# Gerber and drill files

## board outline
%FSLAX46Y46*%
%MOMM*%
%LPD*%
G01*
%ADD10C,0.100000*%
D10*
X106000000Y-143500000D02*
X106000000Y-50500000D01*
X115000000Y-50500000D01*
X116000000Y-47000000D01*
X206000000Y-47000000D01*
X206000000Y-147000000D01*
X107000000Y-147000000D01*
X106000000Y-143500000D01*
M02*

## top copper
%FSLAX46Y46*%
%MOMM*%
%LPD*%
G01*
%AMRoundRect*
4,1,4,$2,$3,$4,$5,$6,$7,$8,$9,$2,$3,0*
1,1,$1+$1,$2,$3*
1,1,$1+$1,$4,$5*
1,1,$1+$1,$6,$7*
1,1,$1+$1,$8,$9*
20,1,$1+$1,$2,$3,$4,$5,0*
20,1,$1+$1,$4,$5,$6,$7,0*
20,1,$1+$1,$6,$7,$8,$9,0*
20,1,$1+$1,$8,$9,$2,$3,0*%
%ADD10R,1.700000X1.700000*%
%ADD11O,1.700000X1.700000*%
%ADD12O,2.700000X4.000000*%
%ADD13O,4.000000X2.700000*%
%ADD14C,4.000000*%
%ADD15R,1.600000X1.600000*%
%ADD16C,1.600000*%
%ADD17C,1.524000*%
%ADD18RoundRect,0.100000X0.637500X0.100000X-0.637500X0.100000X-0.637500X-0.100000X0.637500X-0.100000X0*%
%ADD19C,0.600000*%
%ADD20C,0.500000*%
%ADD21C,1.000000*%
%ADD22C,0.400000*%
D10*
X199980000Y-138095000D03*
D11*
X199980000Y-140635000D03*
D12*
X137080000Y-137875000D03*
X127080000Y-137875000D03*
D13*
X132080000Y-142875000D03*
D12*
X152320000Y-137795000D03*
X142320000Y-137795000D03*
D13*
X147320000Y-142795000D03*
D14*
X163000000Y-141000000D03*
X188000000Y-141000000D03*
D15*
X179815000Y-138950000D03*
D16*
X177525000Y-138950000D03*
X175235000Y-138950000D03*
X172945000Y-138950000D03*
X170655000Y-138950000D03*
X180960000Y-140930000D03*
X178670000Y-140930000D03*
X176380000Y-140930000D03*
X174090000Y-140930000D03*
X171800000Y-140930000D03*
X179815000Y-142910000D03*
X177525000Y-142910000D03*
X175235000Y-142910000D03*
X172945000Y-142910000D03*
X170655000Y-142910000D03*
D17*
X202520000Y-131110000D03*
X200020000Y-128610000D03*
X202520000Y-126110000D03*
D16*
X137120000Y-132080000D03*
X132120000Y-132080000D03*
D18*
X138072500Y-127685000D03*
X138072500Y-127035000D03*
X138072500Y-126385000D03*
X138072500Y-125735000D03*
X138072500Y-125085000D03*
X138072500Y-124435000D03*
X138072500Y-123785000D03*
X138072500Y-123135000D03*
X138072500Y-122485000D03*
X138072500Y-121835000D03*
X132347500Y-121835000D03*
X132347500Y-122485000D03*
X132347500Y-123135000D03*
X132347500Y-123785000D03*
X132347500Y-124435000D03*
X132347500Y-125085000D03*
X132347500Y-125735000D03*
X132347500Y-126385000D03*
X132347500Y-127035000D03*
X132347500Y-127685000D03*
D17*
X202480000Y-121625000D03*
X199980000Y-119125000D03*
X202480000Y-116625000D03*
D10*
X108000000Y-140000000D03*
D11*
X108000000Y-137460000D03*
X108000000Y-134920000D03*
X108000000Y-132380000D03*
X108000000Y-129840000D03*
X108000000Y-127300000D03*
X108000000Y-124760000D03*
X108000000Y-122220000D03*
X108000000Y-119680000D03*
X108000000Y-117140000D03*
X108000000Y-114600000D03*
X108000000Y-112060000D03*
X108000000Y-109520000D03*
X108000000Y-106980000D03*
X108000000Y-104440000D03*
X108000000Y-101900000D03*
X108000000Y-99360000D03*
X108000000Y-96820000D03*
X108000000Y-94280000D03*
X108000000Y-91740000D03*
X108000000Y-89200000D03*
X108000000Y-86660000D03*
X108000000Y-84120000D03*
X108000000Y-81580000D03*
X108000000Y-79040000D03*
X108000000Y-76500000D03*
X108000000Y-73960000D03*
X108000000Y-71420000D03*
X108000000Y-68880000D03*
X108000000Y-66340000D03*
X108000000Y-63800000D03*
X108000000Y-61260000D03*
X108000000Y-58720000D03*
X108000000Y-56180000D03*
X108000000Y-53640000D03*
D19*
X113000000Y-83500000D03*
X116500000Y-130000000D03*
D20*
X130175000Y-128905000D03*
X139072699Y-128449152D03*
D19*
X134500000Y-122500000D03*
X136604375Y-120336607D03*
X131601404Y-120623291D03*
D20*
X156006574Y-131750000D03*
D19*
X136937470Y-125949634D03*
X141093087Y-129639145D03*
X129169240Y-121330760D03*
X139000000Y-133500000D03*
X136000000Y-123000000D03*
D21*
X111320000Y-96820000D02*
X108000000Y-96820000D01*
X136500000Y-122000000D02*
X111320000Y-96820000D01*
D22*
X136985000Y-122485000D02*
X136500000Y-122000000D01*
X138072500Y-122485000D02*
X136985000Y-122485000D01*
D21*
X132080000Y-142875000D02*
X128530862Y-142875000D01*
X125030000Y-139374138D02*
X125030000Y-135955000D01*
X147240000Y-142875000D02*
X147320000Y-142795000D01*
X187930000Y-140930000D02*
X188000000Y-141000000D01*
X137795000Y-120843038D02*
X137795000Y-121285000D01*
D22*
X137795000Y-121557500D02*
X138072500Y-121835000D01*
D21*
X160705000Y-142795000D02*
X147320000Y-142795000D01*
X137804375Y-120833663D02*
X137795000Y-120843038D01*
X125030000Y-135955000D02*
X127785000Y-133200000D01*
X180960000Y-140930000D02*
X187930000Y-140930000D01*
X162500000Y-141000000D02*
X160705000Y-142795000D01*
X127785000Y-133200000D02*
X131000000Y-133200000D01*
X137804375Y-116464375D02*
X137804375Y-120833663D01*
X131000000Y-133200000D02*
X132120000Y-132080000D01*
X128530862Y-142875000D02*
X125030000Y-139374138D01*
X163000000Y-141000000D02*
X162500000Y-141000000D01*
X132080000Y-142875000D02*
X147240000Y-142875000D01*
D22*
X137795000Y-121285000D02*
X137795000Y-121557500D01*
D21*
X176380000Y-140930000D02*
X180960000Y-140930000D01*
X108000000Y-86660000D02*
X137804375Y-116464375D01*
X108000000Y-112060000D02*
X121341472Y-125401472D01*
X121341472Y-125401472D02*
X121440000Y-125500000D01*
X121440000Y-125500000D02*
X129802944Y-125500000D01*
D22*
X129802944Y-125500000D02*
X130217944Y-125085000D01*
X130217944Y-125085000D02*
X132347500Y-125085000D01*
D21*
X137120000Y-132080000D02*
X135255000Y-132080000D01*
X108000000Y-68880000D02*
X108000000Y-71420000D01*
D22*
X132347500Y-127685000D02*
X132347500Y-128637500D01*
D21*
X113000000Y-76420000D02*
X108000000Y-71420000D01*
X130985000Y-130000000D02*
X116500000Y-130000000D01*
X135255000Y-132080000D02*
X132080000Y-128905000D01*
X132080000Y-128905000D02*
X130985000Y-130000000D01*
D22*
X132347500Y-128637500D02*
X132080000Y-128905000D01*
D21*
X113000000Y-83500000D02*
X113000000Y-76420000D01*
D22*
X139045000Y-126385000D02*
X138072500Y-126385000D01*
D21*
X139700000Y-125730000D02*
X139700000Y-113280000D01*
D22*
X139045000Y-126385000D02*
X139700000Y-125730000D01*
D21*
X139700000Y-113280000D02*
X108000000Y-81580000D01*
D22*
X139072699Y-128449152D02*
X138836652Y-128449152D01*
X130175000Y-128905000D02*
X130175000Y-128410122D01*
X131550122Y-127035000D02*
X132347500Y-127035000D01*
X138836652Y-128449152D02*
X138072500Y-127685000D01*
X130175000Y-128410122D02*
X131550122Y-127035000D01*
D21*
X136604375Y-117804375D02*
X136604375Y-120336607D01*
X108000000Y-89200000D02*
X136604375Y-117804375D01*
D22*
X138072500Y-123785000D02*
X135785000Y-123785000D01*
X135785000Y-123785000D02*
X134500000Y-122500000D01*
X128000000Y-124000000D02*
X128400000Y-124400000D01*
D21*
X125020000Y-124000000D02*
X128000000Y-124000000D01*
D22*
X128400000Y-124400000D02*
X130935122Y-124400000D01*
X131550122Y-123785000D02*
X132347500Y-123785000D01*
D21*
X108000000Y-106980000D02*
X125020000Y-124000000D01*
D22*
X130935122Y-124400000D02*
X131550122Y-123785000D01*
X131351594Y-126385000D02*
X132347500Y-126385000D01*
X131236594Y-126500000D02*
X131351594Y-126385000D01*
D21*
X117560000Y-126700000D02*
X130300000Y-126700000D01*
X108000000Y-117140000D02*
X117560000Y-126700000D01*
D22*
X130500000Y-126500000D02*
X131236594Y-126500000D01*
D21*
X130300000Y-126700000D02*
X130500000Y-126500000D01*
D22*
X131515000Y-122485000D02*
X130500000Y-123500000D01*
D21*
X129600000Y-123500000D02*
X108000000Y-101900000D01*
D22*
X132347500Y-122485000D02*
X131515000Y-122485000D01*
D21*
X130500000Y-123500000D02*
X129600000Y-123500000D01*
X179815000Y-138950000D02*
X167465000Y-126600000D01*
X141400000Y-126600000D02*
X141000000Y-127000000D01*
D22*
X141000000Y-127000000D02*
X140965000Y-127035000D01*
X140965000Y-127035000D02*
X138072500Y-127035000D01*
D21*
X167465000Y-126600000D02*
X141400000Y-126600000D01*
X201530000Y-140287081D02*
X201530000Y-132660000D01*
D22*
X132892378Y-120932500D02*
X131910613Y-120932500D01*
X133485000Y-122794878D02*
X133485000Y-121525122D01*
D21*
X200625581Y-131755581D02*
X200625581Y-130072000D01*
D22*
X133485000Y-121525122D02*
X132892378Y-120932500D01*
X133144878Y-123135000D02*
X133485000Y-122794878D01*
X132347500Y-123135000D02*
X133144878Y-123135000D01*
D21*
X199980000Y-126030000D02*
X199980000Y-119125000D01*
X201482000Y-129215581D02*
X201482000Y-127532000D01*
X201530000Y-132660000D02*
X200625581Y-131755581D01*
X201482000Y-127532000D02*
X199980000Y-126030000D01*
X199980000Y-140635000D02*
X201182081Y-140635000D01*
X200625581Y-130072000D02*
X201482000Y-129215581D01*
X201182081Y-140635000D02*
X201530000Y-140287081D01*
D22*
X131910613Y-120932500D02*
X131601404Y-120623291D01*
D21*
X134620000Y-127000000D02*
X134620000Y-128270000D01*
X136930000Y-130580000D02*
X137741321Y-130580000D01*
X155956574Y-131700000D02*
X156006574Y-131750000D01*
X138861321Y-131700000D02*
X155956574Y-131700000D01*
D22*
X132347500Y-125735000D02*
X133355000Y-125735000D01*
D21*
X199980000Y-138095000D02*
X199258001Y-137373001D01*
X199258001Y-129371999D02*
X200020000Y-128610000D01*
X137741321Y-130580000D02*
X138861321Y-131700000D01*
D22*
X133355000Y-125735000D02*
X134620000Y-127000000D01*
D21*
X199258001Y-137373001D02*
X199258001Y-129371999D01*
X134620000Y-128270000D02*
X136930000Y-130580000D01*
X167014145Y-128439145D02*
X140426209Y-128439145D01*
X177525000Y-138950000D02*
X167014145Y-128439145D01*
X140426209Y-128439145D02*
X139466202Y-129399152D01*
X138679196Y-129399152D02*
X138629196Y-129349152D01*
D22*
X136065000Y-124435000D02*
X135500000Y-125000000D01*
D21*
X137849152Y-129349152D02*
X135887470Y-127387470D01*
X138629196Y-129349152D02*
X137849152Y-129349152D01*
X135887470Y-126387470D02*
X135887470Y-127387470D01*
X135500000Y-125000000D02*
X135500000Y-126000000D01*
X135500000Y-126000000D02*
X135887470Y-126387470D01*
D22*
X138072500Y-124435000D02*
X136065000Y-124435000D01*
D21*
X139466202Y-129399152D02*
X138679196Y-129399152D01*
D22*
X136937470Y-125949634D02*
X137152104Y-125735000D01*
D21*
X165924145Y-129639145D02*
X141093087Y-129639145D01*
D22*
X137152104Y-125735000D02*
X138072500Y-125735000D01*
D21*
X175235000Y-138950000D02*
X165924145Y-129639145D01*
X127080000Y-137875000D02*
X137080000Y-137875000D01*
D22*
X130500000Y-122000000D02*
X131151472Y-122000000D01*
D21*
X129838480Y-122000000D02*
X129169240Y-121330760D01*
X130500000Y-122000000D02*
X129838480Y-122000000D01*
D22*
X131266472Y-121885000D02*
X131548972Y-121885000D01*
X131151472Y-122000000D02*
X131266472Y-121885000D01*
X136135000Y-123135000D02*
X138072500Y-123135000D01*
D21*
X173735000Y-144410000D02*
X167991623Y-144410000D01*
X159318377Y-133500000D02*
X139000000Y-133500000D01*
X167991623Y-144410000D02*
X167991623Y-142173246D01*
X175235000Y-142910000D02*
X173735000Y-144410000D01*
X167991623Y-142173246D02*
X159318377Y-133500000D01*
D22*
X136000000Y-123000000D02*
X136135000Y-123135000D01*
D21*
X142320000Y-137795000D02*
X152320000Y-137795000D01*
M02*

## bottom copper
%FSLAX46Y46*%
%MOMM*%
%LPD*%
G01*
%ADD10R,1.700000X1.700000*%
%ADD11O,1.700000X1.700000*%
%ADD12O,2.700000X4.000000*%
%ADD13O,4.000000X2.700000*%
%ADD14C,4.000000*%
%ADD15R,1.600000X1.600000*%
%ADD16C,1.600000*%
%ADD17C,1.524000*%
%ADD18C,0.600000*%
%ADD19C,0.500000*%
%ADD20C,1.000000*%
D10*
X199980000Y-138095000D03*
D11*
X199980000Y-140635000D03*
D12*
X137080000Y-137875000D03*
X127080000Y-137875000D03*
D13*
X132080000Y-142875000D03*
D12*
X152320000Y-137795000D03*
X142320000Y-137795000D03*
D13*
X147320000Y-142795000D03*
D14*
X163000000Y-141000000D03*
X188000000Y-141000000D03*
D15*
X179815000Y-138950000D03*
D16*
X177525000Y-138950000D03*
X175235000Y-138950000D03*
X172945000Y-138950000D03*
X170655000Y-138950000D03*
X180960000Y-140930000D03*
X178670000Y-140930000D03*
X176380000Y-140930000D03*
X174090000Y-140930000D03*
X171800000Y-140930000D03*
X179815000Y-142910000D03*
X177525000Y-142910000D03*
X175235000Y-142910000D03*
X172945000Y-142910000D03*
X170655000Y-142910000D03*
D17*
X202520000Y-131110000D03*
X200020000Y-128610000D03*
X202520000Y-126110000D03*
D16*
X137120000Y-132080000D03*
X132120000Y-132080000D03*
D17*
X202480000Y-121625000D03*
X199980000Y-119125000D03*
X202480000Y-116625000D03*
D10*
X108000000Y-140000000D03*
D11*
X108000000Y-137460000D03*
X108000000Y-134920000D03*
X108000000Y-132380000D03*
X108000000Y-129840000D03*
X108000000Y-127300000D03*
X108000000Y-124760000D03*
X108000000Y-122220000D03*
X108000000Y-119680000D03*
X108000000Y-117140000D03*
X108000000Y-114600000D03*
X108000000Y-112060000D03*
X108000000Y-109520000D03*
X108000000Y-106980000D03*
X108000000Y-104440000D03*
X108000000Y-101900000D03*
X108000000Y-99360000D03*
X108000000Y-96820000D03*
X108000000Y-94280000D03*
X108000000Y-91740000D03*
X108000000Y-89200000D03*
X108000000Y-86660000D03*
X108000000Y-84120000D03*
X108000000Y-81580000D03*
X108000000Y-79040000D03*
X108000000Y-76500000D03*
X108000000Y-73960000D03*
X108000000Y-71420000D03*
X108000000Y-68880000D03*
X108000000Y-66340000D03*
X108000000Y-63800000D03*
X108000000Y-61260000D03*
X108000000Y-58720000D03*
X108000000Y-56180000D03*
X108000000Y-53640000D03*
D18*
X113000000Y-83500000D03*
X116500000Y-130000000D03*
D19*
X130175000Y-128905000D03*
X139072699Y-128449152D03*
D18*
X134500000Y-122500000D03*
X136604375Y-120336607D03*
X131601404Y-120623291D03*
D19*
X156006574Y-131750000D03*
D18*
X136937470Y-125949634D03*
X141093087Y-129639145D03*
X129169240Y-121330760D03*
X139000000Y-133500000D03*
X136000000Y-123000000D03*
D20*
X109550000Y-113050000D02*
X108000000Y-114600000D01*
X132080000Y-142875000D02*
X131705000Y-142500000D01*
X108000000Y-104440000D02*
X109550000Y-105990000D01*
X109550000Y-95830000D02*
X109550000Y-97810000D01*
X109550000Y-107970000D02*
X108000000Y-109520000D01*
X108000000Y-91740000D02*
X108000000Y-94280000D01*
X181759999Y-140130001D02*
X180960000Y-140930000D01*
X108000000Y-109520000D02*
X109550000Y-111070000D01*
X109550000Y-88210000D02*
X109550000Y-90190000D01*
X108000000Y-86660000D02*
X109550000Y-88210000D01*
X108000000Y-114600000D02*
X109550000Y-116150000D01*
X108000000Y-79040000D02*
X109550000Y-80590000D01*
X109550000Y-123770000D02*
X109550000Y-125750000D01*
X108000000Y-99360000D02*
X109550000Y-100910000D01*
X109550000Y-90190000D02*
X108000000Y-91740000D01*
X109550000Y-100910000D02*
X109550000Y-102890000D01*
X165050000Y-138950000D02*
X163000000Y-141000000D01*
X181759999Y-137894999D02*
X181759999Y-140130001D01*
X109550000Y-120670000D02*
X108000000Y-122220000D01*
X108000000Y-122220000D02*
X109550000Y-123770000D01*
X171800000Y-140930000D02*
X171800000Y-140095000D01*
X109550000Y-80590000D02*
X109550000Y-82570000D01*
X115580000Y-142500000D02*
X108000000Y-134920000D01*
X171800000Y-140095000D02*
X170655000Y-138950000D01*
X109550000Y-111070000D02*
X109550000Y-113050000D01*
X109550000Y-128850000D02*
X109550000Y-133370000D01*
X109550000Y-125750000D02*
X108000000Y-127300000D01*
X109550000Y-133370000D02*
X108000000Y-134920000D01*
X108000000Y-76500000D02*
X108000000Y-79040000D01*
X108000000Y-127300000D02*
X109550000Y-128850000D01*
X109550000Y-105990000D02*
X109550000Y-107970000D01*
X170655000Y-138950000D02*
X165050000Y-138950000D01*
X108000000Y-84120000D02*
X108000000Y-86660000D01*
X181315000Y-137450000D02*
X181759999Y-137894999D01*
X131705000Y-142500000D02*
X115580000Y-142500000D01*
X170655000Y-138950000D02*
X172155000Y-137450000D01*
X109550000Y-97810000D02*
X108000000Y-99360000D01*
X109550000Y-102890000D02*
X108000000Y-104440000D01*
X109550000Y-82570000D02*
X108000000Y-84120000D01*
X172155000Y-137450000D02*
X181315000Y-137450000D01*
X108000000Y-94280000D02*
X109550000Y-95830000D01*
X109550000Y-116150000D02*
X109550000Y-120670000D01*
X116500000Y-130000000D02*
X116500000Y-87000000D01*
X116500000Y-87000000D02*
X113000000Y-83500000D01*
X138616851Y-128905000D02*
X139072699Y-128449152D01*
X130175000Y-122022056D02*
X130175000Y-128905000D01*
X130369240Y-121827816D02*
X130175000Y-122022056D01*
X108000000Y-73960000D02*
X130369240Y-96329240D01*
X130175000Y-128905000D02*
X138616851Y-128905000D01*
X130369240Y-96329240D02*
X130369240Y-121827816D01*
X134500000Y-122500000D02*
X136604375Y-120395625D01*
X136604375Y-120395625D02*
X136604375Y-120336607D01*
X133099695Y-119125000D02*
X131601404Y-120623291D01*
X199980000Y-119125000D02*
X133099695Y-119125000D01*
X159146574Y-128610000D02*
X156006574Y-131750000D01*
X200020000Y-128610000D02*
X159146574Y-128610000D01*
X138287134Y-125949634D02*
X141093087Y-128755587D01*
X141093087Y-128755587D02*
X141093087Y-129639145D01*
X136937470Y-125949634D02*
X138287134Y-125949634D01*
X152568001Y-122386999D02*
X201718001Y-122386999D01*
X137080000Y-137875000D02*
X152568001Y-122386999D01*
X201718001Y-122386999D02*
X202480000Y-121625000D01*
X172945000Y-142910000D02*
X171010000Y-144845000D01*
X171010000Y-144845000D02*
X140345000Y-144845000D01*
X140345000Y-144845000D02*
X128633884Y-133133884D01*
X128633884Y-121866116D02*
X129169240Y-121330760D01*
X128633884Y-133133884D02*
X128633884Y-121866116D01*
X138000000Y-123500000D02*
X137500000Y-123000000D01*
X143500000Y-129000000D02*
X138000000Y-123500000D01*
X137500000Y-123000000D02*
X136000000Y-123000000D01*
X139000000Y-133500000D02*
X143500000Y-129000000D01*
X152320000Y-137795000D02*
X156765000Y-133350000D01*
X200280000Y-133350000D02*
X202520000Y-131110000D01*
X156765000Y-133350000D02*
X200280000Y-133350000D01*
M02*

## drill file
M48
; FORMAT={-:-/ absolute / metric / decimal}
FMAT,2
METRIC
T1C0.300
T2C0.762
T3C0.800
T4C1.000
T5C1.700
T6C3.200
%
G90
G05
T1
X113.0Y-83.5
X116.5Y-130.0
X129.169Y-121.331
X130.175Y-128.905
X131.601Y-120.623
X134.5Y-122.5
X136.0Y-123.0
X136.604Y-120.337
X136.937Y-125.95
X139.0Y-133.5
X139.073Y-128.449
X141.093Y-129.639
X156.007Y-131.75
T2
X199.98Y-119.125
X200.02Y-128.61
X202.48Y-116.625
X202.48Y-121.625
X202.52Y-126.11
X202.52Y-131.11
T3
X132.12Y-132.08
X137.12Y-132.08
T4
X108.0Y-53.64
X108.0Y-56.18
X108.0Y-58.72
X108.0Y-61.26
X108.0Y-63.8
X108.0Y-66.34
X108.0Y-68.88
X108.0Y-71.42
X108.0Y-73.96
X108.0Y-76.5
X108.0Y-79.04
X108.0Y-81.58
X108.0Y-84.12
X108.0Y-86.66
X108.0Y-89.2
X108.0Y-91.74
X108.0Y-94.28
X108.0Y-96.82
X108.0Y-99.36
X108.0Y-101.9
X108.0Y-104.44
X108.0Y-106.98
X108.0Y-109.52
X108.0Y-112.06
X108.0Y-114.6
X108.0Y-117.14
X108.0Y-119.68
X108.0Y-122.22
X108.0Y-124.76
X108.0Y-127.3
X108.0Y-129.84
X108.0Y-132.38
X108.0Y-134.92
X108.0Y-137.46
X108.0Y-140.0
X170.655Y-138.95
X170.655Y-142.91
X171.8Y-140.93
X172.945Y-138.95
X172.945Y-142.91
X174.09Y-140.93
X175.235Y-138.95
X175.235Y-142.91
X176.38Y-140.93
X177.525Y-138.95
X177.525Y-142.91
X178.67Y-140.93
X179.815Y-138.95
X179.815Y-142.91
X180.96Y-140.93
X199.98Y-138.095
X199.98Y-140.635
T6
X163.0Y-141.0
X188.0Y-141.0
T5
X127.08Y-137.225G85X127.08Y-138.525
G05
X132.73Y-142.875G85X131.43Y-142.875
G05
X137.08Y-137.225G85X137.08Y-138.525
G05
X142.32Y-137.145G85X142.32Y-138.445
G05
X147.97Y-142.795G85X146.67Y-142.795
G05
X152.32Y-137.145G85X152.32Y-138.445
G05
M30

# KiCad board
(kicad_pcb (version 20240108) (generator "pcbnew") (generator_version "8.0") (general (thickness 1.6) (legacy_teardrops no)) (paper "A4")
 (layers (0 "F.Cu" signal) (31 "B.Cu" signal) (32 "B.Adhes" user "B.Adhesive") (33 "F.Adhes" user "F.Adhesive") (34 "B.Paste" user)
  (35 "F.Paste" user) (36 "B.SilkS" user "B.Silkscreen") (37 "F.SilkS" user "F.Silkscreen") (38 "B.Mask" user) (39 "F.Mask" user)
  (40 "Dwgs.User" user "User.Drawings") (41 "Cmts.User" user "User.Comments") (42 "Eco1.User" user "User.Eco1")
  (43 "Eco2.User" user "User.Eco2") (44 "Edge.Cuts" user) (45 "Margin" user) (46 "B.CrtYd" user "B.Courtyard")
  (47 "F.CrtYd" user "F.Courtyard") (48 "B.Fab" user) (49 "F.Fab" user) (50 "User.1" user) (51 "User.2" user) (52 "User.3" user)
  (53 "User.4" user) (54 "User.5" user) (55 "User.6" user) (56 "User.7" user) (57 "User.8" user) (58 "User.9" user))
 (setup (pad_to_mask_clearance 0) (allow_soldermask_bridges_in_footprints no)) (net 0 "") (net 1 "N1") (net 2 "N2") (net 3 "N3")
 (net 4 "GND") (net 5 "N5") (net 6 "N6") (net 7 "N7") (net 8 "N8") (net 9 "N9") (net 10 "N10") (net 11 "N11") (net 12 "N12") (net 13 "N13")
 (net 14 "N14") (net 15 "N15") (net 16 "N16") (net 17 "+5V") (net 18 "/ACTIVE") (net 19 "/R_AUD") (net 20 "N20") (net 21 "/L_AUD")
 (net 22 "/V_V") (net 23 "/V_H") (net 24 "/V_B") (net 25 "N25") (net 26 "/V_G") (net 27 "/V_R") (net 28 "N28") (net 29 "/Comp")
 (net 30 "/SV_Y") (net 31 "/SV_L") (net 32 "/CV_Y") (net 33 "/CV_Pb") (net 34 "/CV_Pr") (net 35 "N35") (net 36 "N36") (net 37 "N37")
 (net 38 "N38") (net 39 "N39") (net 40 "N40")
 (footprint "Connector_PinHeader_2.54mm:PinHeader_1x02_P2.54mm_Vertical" (layer "F.Cu") (at 199.98 138.095)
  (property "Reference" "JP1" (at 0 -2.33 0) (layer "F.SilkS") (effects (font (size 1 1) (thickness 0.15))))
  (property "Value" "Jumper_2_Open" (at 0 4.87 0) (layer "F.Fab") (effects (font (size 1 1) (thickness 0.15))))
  (pad "1" thru_hole rect (at 0 0) (size 1.7 1.7) (drill 1) (layers "*.Cu" "*.Mask") (remove_unused_layers no) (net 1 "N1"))
  (pad "2" thru_hole oval (at 0 2.54) (size 1.7 1.7) (drill 1) (layers "*.Cu" "*.Mask") (remove_unused_layers no) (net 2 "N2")))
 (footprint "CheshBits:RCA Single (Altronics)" (layer "F.Cu") (at 132.08 137.875 180)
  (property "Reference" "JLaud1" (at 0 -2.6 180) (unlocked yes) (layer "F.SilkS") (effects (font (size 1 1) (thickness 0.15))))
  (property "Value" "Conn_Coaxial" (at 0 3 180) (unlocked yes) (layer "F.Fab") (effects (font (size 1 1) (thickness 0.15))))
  (pad "1" thru_hole oval (at -5 0 270) (size 4 2.7) (drill oval 3 1.7) (layers "*.Cu" "*.Mask") (remove_unused_layers no) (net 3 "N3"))
  (pad "1" thru_hole oval (at 5 0 270) (size 4 2.7) (drill oval 3 1.7) (layers "*.Cu" "*.Mask") (remove_unused_layers no) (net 3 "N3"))
  (pad "2" thru_hole oval (at 0 -5 180) (size 4 2.7) (drill oval 3 1.7) (layers "*.Cu" "*.Mask") (remove_unused_layers no) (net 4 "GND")))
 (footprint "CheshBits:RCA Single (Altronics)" (layer "F.Cu") (at 147.32 137.795 180)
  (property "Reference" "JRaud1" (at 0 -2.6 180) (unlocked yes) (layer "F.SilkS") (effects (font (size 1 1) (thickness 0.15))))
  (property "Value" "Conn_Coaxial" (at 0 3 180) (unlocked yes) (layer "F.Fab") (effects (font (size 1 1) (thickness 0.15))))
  (pad "1" thru_hole oval (at -5 0 270) (size 4 2.7) (drill oval 3 1.7) (layers "*.Cu" "*.Mask") (remove_unused_layers no) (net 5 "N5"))
  (pad "1" thru_hole oval (at 5 0 270) (size 4 2.7) (drill oval 3 1.7) (layers "*.Cu" "*.Mask") (remove_unused_layers no) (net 5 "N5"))
  (pad "2" thru_hole oval (at 0 -5 180) (size 4 2.7) (drill oval 3 1.7) (layers "*.Cu" "*.Mask") (remove_unused_layers no) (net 4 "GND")))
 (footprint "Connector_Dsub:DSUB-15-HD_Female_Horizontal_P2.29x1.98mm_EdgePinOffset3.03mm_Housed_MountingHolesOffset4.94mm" (layer "F.Cu")
  (at 179.815 138.95)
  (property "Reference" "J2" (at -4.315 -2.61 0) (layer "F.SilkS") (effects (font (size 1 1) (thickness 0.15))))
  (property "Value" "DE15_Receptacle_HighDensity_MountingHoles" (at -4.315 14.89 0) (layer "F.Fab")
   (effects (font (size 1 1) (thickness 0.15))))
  (pad "0" thru_hole circle (at -16.815 2.05) (size 4 4) (drill 3.2) (layers "*.Cu" "*.Mask") (remove_unused_layers no) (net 4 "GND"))
  (pad "0" thru_hole circle (at 8.185 2.05) (size 4 4) (drill 3.2) (layers "*.Cu" "*.Mask") (remove_unused_layers no) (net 4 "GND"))
  (pad "1" thru_hole rect (at 0 0) (size 1.6 1.6) (drill 1) (layers "*.Cu" "*.Mask") (remove_unused_layers no) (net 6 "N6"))
  (pad "2" thru_hole circle (at -2.29 0) (size 1.6 1.6) (drill 1) (layers "*.Cu" "*.Mask") (remove_unused_layers no) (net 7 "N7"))
  (pad "3" thru_hole circle (at -4.58 0) (size 1.6 1.6) (drill 1) (layers "*.Cu" "*.Mask") (remove_unused_layers no) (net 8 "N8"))
  (pad "4" thru_hole circle (at -6.87 0) (size 1.6 1.6) (drill 1) (layers "*.Cu" "*.Mask") (remove_unused_layers no) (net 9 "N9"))
  (pad "5" thru_hole circle (at -9.16 0) (size 1.6 1.6) (drill 1) (layers "*.Cu" "*.Mask") (remove_unused_layers no) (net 4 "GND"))
  (pad "6" thru_hole circle (at 1.145 1.98) (size 1.6 1.6) (drill 1) (layers "*.Cu" "*.Mask") (remove_unused_layers no) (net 4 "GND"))
  (pad "7" thru_hole circle (at -1.145 1.98) (size 1.6 1.6) (drill 1) (layers "*.Cu" "*.Mask") (remove_unused_layers no) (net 4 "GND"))
  (pad "8" thru_hole circle (at -3.435 1.98) (size 1.6 1.6) (drill 1) (layers "*.Cu" "*.Mask") (remove_unused_layers no) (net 4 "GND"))
  (pad "9" thru_hole circle (at -5.725 1.98) (size 1.6 1.6) (drill 1) (layers "*.Cu" "*.Mask") (remove_unused_layers no) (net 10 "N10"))
  (pad "10" thru_hole circle (at -8.015 1.98) (size 1.6 1.6) (drill 1) (layers "*.Cu" "*.Mask") (remove_unused_layers no) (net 4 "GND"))
  (pad "11" thru_hole circle (at 0 3.96) (size 1.6 1.6) (drill 1) (layers "*.Cu" "*.Mask") (remove_unused_layers no) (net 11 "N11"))
  (pad "12" thru_hole circle (at -2.29 3.96) (size 1.6 1.6) (drill 1) (layers "*.Cu" "*.Mask") (remove_unused_layers no) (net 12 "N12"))
  (pad "13" thru_hole circle (at -4.58 3.96) (size 1.6 1.6) (drill 1) (layers "*.Cu" "*.Mask") (remove_unused_layers no) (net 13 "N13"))
  (pad "14" thru_hole circle (at -6.87 3.96) (size 1.6 1.6) (drill 1) (layers "*.Cu" "*.Mask") (remove_unused_layers no) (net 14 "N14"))
  (pad "15" thru_hole circle (at -9.16 3.96) (size 1.6 1.6) (drill 1) (layers "*.Cu" "*.Mask") (remove_unused_layers no) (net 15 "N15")))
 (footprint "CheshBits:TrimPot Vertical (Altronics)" (layer "F.Cu") (at 193.62 128.61 90)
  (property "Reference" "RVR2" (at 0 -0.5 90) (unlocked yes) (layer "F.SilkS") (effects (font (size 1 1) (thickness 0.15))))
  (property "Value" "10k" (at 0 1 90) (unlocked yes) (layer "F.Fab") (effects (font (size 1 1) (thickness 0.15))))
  (pad "1" thru_hole circle (at -2.5 8.9 90) (size 1.524 1.524) (drill 0.762) (layers "*.Cu" "*.Mask") (remove_unused_layers no)
   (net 5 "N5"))
  (pad "2" thru_hole circle (at 0 6.4 90) (size 1.524 1.524) (drill 0.762) (layers "*.Cu" "*.Mask") (remove_unused_layers no) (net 1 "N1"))
  (pad "3" thru_hole circle (at 2.5 8.9 90) (size 1.524 1.524) (drill 0.762) (layers "*.Cu" "*.Mask") (remove_unused_layers no)
   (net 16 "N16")))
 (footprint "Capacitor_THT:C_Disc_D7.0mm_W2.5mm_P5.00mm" (layer "F.Cu") (at 137.12 132.08 180)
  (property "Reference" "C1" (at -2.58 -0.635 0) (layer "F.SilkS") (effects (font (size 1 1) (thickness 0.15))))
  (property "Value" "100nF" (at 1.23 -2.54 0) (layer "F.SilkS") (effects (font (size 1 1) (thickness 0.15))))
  (pad "1" thru_hole circle (at 0 0 180) (size 1.6 1.6) (drill 0.8) (layers "*.Cu" "*.Mask") (remove_unused_layers no) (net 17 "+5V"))
  (pad "2" thru_hole circle (at 5 0 180) (size 1.6 1.6) (drill 0.8) (layers "*.Cu" "*.Mask") (remove_unused_layers no) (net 4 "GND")))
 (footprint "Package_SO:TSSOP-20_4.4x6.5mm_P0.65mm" (layer "F.Cu") (at 135.21 124.76 180)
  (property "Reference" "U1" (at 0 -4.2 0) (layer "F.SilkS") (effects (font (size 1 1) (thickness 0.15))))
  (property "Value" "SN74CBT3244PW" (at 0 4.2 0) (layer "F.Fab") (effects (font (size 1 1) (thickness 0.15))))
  (pad "1" smd roundrect (at -2.8625 -2.925 180) (size 1.475 0.4) (layers "F.Cu" "F.Paste" "F.Mask") (roundrect_rratio 0.25)
   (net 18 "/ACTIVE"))
  (pad "2" smd roundrect (at -2.8625 -2.275 180) (size 1.475 0.4) (layers "F.Cu" "F.Paste" "F.Mask") (roundrect_rratio 0.25) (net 6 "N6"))
  (pad "3" smd roundrect (at -2.8625 -1.625 180) (size 1.475 0.4) (layers "F.Cu" "F.Paste" "F.Mask") (roundrect_rratio 0.25)
   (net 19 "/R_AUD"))
  (pad "4" smd roundrect (at -2.8625 -0.975 180) (size 1.475 0.4) (layers "F.Cu" "F.Paste" "F.Mask") (roundrect_rratio 0.25) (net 8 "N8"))
  (pad "5" smd roundrect (at -2.8625 -0.325 180) (size 1.475 0.4) (layers "F.Cu" "F.Paste" "F.Mask") (roundrect_rratio 0.25) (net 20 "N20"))
  (pad "6" smd roundrect (at -2.8625 0.325 180) (size 1.475 0.4) (layers "F.Cu" "F.Paste" "F.Mask") (roundrect_rratio 0.25) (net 7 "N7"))
  (pad "7" smd roundrect (at -2.8625 0.975 180) (size 1.475 0.4) (layers "F.Cu" "F.Paste" "F.Mask") (roundrect_rratio 0.25)
   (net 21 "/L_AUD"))
  (pad "8" smd roundrect (at -2.8625 1.625 180) (size 1.475 0.4) (layers "F.Cu" "F.Paste" "F.Mask") (roundrect_rratio 0.25) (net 13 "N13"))
  (pad "9" smd roundrect (at -2.8625 2.275 180) (size 1.475 0.4) (layers "F.Cu" "F.Paste" "F.Mask") (roundrect_rratio 0.25) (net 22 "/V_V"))
  (pad "10" smd roundrect (at -2.8625 2.925 180) (size 1.475 0.4) (layers "F.Cu" "F.Paste" "F.Mask") (roundrect_rratio 0.25) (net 4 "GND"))
  (pad "11" smd roundrect (at 2.8625 2.925 180) (size 1.475 0.4) (layers "F.Cu" "F.Paste" "F.Mask") (roundrect_rratio 0.25) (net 14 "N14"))
  (pad "12" smd roundrect (at 2.8625 2.275 180) (size 1.475 0.4) (layers "F.Cu" "F.Paste" "F.Mask") (roundrect_rratio 0.25) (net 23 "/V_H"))
  (pad "13" smd roundrect (at 2.8625 1.625 180) (size 1.475 0.4) (layers "F.Cu" "F.Paste" "F.Mask") (roundrect_rratio 0.25) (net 2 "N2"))
  (pad "14" smd roundrect (at 2.8625 0.975 180) (size 1.475 0.4) (layers "F.Cu" "F.Paste" "F.Mask") (roundrect_rratio 0.25) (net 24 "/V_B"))
  (pad "15" smd roundrect (at 2.8625 0.325 180) (size 1.475 0.4) (layers "F.Cu" "F.Paste" "F.Mask") (roundrect_rratio 0.25) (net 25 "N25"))
  (pad "16" smd roundrect (at 2.8625 -0.325 180) (size 1.475 0.4) (layers "F.Cu" "F.Paste" "F.Mask") (roundrect_rratio 0.25) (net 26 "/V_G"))
  (pad "17" smd roundrect (at 2.8625 -0.975 180) (size 1.475 0.4) (layers "F.Cu" "F.Paste" "F.Mask") (roundrect_rratio 0.25) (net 1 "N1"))
  (pad "18" smd roundrect (at 2.8625 -1.625 180) (size 1.475 0.4) (layers "F.Cu" "F.Paste" "F.Mask") (roundrect_rratio 0.25) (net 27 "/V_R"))
  (pad "19" smd roundrect (at 2.8625 -2.275 180) (size 1.475 0.4) (layers "F.Cu" "F.Paste" "F.Mask") (roundrect_rratio 0.25)
   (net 18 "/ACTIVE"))
  (pad "20" smd roundrect (at 2.8625 -2.925 180) (size 1.475 0.4) (layers "F.Cu" "F.Paste" "F.Mask") (roundrect_rratio 0.25) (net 17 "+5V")))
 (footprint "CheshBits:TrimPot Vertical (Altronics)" (layer "F.Cu") (at 193.58 119.125 90)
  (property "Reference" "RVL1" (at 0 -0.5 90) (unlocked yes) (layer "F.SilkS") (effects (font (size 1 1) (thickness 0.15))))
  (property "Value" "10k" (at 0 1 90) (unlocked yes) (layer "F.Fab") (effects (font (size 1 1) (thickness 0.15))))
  (pad "1" thru_hole circle (at -2.5 8.9 90) (size 1.524 1.524) (drill 0.762) (layers "*.Cu" "*.Mask") (remove_unused_layers no)
   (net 3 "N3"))
  (pad "2" thru_hole circle (at 0 6.4 90) (size 1.524 1.524) (drill 0.762) (layers "*.Cu" "*.Mask") (remove_unused_layers no) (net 2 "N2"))
  (pad "3" thru_hole circle (at 2.5 8.9 90) (size 1.524 1.524) (drill 0.762) (layers "*.Cu" "*.Mask") (remove_unused_layers no)
   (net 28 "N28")))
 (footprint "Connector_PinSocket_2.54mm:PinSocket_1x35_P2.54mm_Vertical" (layer "B.Cu") (at 108 140)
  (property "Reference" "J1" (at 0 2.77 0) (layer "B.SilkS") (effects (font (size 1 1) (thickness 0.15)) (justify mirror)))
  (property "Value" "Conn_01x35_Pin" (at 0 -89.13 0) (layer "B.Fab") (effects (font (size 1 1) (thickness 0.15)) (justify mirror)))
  (pad "1" thru_hole rect (at 0 0) (size 1.7 1.7) (drill 1) (layers "*.Cu" "*.Mask") (remove_unused_layers no) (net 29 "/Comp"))
  (pad "2" thru_hole oval (at 0 -2.54) (size 1.7 1.7) (drill 1) (layers "*.Cu" "*.Mask") (remove_unused_layers no) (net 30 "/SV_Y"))
  (pad "3" thru_hole oval (at 0 -5.08) (size 1.7 1.7) (drill 1) (layers "*.Cu" "*.Mask") (remove_unused_layers no) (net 4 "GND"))
  (pad "4" thru_hole oval (at 0 -7.62) (size 1.7 1.7) (drill 1) (layers "*.Cu" "*.Mask") (remove_unused_layers no) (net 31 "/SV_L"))
  (pad "5" thru_hole oval (at 0 -10.16) (size 1.7 1.7) (drill 1) (layers "*.Cu" "*.Mask") (remove_unused_layers no) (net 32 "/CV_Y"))
  (pad "6" thru_hole oval (at 0 -12.7) (size 1.7 1.7) (drill 1) (layers "*.Cu" "*.Mask") (remove_unused_layers no) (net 4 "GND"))
  (pad "7" thru_hole oval (at 0 -15.24) (size 1.7 1.7) (drill 1) (layers "*.Cu" "*.Mask") (remove_unused_layers no) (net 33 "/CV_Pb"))
  (pad "8" thru_hole oval (at 0 -17.78) (size 1.7 1.7) (drill 1) (layers "*.Cu" "*.Mask") (remove_unused_layers no) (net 4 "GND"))
  (pad "9" thru_hole oval (at 0 -20.32) (size 1.7 1.7) (drill 1) (layers "*.Cu" "*.Mask") (remove_unused_layers no) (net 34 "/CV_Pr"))
  (pad "10" thru_hole oval (at 0 -22.86) (size 1.7 1.7) (drill 1) (layers "*.Cu" "*.Mask") (remove_unused_layers no) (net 27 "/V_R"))
  (pad "11" thru_hole oval (at 0 -25.4) (size 1.7 1.7) (drill 1) (layers "*.Cu" "*.Mask") (remove_unused_layers no) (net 4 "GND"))
  (pad "12" thru_hole oval (at 0 -27.94) (size 1.7 1.7) (drill 1) (layers "*.Cu" "*.Mask") (remove_unused_layers no) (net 26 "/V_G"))
  (pad "13" thru_hole oval (at 0 -30.48) (size 1.7 1.7) (drill 1) (layers "*.Cu" "*.Mask") (remove_unused_layers no) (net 4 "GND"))
  (pad "14" thru_hole oval (at 0 -33.02) (size 1.7 1.7) (drill 1) (layers "*.Cu" "*.Mask") (remove_unused_layers no) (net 24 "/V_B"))
  (pad "15" thru_hole oval (at 0 -35.56) (size 1.7 1.7) (drill 1) (layers "*.Cu" "*.Mask") (remove_unused_layers no) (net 4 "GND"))
  (pad "16" thru_hole oval (at 0 -38.1) (size 1.7 1.7) (drill 1) (layers "*.Cu" "*.Mask") (remove_unused_layers no) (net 23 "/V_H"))
  (pad "17" thru_hole oval (at 0 -40.64) (size 1.7 1.7) (drill 1) (layers "*.Cu" "*.Mask") (remove_unused_layers no) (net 4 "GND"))
  (pad "18" thru_hole oval (at 0 -43.18) (size 1.7 1.7) (drill 1) (layers "*.Cu" "*.Mask") (remove_unused_layers no) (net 22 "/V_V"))
  (pad "19" thru_hole oval (at 0 -45.72) (size 1.7 1.7) (drill 1) (layers "*.Cu" "*.Mask") (remove_unused_layers no) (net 4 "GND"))
  (pad "20" thru_hole oval (at 0 -48.26) (size 1.7 1.7) (drill 1) (layers "*.Cu" "*.Mask") (remove_unused_layers no) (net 4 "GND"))
  (pad "21" thru_hole oval (at 0 -50.8) (size 1.7 1.7) (drill 1) (layers "*.Cu" "*.Mask") (remove_unused_layers no) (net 21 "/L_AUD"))
  (pad "22" thru_hole oval (at 0 -53.34) (size 1.7 1.7) (drill 1) (layers "*.Cu" "*.Mask") (remove_unused_layers no) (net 4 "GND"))
  (pad "23" thru_hole oval (at 0 -55.88) (size 1.7 1.7) (drill 1) (layers "*.Cu" "*.Mask") (remove_unused_layers no) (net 4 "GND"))
  (pad "24" thru_hole oval (at 0 -58.42) (size 1.7 1.7) (drill 1) (layers "*.Cu" "*.Mask") (remove_unused_layers no) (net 19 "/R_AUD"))
  (pad "25" thru_hole oval (at 0 -60.96) (size 1.7 1.7) (drill 1) (layers "*.Cu" "*.Mask") (remove_unused_layers no) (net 4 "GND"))
  (pad "26" thru_hole oval (at 0 -63.5) (size 1.7 1.7) (drill 1) (layers "*.Cu" "*.Mask") (remove_unused_layers no) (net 4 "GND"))
  (pad "27" thru_hole oval (at 0 -66.04) (size 1.7 1.7) (drill 1) (layers "*.Cu" "*.Mask") (remove_unused_layers no) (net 18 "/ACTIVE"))
  (pad "28" thru_hole oval (at 0 -68.58) (size 1.7 1.7) (drill 1) (layers "*.Cu" "*.Mask") (remove_unused_layers no) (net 17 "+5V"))
  (pad "29" thru_hole oval (at 0 -71.12) (size 1.7 1.7) (drill 1) (layers "*.Cu" "*.Mask") (remove_unused_layers no) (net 17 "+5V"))
  (pad "30" thru_hole oval (at 0 -73.66) (size 1.7 1.7) (drill 1) (layers "*.Cu" "*.Mask") (remove_unused_layers no) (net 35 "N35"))
  (pad "31" thru_hole oval (at 0 -76.2) (size 1.7 1.7) (drill 1) (layers "*.Cu" "*.Mask") (remove_unused_layers no) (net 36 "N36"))
  (pad "32" thru_hole oval (at 0 -78.74) (size 1.7 1.7) (drill 1) (layers "*.Cu" "*.Mask") (remove_unused_layers no) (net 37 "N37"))
  (pad "33" thru_hole oval (at 0 -81.28) (size 1.7 1.7) (drill 1) (layers "*.Cu" "*.Mask") (remove_unused_layers no) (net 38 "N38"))
  (pad "34" thru_hole oval (at 0 -83.82) (size 1.7 1.7) (drill 1) (layers "*.Cu" "*.Mask") (remove_unused_layers no) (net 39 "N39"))
  (pad "35" thru_hole oval (at 0 -86.36) (size 1.7 1.7) (drill 1) (layers "*.Cu" "*.Mask") (remove_unused_layers no) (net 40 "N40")))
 (gr_poly
  (pts (xy 106 143.5) (xy 106 50.5) (xy 115 50.5) (xy 116 47) (xy 206 47) (xy 206 147) (xy 107 147)) (stroke (width 0.1) (type solid))
  (fill none) (layer "Edge.Cuts"))
 (segment (start 111.32 96.82) (end 108 96.82) (width 1) (layer "F.Cu") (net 22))
 (segment (start 136.5 122) (end 111.32 96.82) (width 1) (layer "F.Cu") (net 22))
 (segment (start 136.985 122.485) (end 136.5 122) (width 0.4) (layer "F.Cu") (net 22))
 (segment (start 138.0725 122.485) (end 136.985 122.485) (width 0.4) (layer "F.Cu") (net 22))
 (segment (start 132.08 142.875) (end 128.530862 142.875) (width 1) (layer "F.Cu") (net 4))
 (segment (start 125.03 139.374138) (end 125.03 135.955) (width 1) (layer "F.Cu") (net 4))
 (segment (start 147.24 142.875) (end 147.32 142.795) (width 1) (layer "F.Cu") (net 4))
 (segment (start 187.93 140.93) (end 188 141) (width 1) (layer "F.Cu") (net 4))
 (segment (start 137.795 120.843038) (end 137.795 121.285) (width 1) (layer "F.Cu") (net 4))
 (segment (start 137.795 121.5575) (end 138.0725 121.835) (width 0.4) (layer "F.Cu") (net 4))
 (segment (start 160.705 142.795) (end 147.32 142.795) (width 1) (layer "F.Cu") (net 4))
 (segment (start 137.804375 120.833663) (end 137.795 120.843038) (width 1) (layer "F.Cu") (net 4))
 (segment (start 125.03 135.955) (end 127.785 133.2) (width 1) (layer "F.Cu") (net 4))
 (segment (start 180.96 140.93) (end 187.93 140.93) (width 1) (layer "F.Cu") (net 4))
 (segment (start 162.5 141) (end 160.705 142.795) (width 1) (layer "F.Cu") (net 4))
 (segment (start 127.785 133.2) (end 131 133.2) (width 1) (layer "F.Cu") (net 4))
 (segment (start 137.804375 116.464375) (end 137.804375 120.833663) (width 1) (layer "F.Cu") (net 4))
 (segment (start 131 133.2) (end 132.12 132.08) (width 1) (layer "F.Cu") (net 4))
 (segment (start 128.530862 142.875) (end 125.03 139.374138) (width 1) (layer "F.Cu") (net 4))
 (segment (start 163 141) (end 162.5 141) (width 1) (layer "F.Cu") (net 4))
 (segment (start 132.08 142.875) (end 147.24 142.875) (width 1) (layer "F.Cu") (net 4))
 (segment (start 137.795 121.285) (end 137.795 121.5575) (width 0.4) (layer "F.Cu") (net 4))
 (segment (start 176.38 140.93) (end 180.96 140.93) (width 1) (layer "F.Cu") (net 4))
 (segment (start 108 86.66) (end 137.804375 116.464375) (width 1) (layer "F.Cu") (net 4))
 (segment (start 109.55 113.05) (end 108 114.6) (width 1) (layer "B.Cu") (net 4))
 (segment (start 132.08 142.875) (end 131.705 142.5) (width 1) (layer "B.Cu") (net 4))
 (segment (start 108 104.44) (end 109.55 105.99) (width 1) (layer "B.Cu") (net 4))
 (segment (start 109.55 95.83) (end 109.55 97.81) (width 1) (layer "B.Cu") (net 4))
 (segment (start 109.55 107.97) (end 108 109.52) (width 1) (layer "B.Cu") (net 4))
 (segment (start 108 91.74) (end 108 94.28) (width 1) (layer "B.Cu") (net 4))
 (segment (start 181.759999 140.130001) (end 180.96 140.93) (width 1) (layer "B.Cu") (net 4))
 (segment (start 108 109.52) (end 109.55 111.07) (width 1) (layer "B.Cu") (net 4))
 (segment (start 109.55 88.21) (end 109.55 90.19) (width 1) (layer "B.Cu") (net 4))
 (segment (start 108 86.66) (end 109.55 88.21) (width 1) (layer "B.Cu") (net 4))
 (segment (start 108 114.6) (end 109.55 116.15) (width 1) (layer "B.Cu") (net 4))
 (segment (start 108 79.04) (end 109.55 80.59) (width 1) (layer "B.Cu") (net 4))
 (segment (start 109.55 123.77) (end 109.55 125.75) (width 1) (layer "B.Cu") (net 4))
 (segment (start 108 99.36) (end 109.55 100.91) (width 1) (layer "B.Cu") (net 4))
 (segment (start 109.55 90.19) (end 108 91.74) (width 1) (layer "B.Cu") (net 4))
 (segment (start 109.55 100.91) (end 109.55 102.89) (width 1) (layer "B.Cu") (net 4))
 (segment (start 165.05 138.95) (end 163 141) (width 1) (layer "B.Cu") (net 4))
 (segment (start 181.759999 137.894999) (end 181.759999 140.130001) (width 1) (layer "B.Cu") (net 4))
 (segment (start 109.55 120.67) (end 108 122.22) (width 1) (layer "B.Cu") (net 4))
 (segment (start 108 122.22) (end 109.55 123.77) (width 1) (layer "B.Cu") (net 4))
 (segment (start 171.8 140.93) (end 171.8 140.095) (width 1) (layer "B.Cu") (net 4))
 (segment (start 109.55 80.59) (end 109.55 82.57) (width 1) (layer "B.Cu") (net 4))
 (segment (start 115.58 142.5) (end 108 134.92) (width 1) (layer "B.Cu") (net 4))
 (segment (start 171.8 140.095) (end 170.655 138.95) (width 1) (layer "B.Cu") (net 4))
 (segment (start 109.55 111.07) (end 109.55 113.05) (width 1) (layer "B.Cu") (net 4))
 (segment (start 109.55 128.85) (end 109.55 133.37) (width 1) (layer "B.Cu") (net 4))
 (segment (start 109.55 125.75) (end 108 127.3) (width 1) (layer "B.Cu") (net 4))
 (segment (start 109.55 133.37) (end 108 134.92) (width 1) (layer "B.Cu") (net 4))
 (segment (start 108 76.5) (end 108 79.04) (width 1) (layer "B.Cu") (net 4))
 (segment (start 108 127.3) (end 109.55 128.85) (width 1) (layer "B.Cu") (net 4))
 (segment (start 109.55 105.99) (end 109.55 107.97) (width 1) (layer "B.Cu") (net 4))
 (segment (start 170.655 138.95) (end 165.05 138.95) (width 1) (layer "B.Cu") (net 4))
 (segment (start 108 84.12) (end 108 86.66) (width 1) (layer "B.Cu") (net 4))
 (segment (start 181.315 137.45) (end 181.759999 137.894999) (width 1) (layer "B.Cu") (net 4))
 (segment (start 131.705 142.5) (end 115.58 142.5) (width 1) (layer "B.Cu") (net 4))
 (segment (start 170.655 138.95) (end 172.155 137.45) (width 1) (layer "B.Cu") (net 4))
 (segment (start 109.55 97.81) (end 108 99.36) (width 1) (layer "B.Cu") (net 4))
 (segment (start 109.55 102.89) (end 108 104.44) (width 1) (layer "B.Cu") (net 4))
 (segment (start 109.55 82.57) (end 108 84.12) (width 1) (layer "B.Cu") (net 4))
 (segment (start 172.155 137.45) (end 181.315 137.45) (width 1) (layer "B.Cu") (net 4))
 (segment (start 108 94.28) (end 109.55 95.83) (width 1) (layer "B.Cu") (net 4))
 (segment (start 109.55 116.15) (end 109.55 120.67) (width 1) (layer "B.Cu") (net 4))
 (segment (start 108 112.06) (end 121.341472 125.401472) (width 1) (layer "F.Cu") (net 26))
 (segment (start 121.341472 125.401472) (end 121.44 125.5) (width 1) (layer "F.Cu") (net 26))
 (segment (start 121.44 125.5) (end 129.802944 125.5) (width 1) (layer "F.Cu") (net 26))
 (segment (start 129.802944 125.5) (end 130.217944 125.085) (width 0.4) (layer "F.Cu") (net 26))
 (segment (start 130.217944 125.085) (end 132.3475 125.085) (width 0.4) (layer "F.Cu") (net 26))
 (segment (start 137.12 132.08) (end 135.255 132.08) (width 1) (layer "F.Cu") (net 17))
 (segment (start 108 68.88) (end 108 71.42) (width 1) (layer "F.Cu") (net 17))
 (segment (start 132.3475 127.685) (end 132.3475 128.6375) (width 0.4) (layer "F.Cu") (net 17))
 (segment (start 113 76.42) (end 108 71.42) (width 1) (layer "F.Cu") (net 17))
 (segment (start 130.985 130) (end 116.5 130) (width 1) (layer "F.Cu") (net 17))
 (segment (start 135.255 132.08) (end 132.08 128.905) (width 1) (layer "F.Cu") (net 17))
 (segment (start 132.08 128.905) (end 130.985 130) (width 1) (layer "F.Cu") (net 17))
 (segment (start 132.3475 128.6375) (end 132.08 128.905) (width 0.4) (layer "F.Cu") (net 17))
 (segment (start 113 83.5) (end 113 76.42) (width 1) (layer "F.Cu") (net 17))
 (via (at 113 83.5) (size 0.6) (drill 0.3) (layers "F.Cu" "B.Cu") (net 17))
 (via (at 116.5 130) (size 0.6) (drill 0.3) (layers "F.Cu" "B.Cu") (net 17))
 (segment (start 116.5 130) (end 116.5 87) (width 1) (layer "B.Cu") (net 17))
 (segment (start 116.5 87) (end 113 83.5) (width 1) (layer "B.Cu") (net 17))
 (segment (start 139.045 126.385) (end 138.0725 126.385) (width 0.4) (layer "F.Cu") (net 19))
 (segment (start 139.7 125.73) (end 139.7 113.28) (width 1) (layer "F.Cu") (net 19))
 (segment (start 139.045 126.385) (end 139.7 125.73) (width 0.4) (layer "F.Cu") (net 19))
 (segment (start 139.7 113.28) (end 108 81.58) (width 1) (layer "F.Cu") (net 19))
 (segment (start 139.072699 128.449152) (end 138.836652 128.449152) (width 0.4) (layer "F.Cu") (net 18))
 (segment (start 130.175 128.905) (end 130.175 128.410122) (width 0.4) (layer "F.Cu") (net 18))
 (segment (start 131.550122 127.035) (end 132.3475 127.035) (width 0.4) (layer "F.Cu") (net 18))
 (segment (start 138.836652 128.449152) (end 138.0725 127.685) (width 0.4) (layer "F.Cu") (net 18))
 (segment (start 130.175 128.410122) (end 131.550122 127.035) (width 0.4) (layer "F.Cu") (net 18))
 (via (at 130.175 128.905) (size 0.5) (drill 0.3) (layers "F.Cu" "B.Cu") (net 18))
 (via (at 139.072699 128.449152) (size 0.5) (drill 0.3) (layers "F.Cu" "B.Cu") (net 18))
 (segment (start 138.616851 128.905) (end 139.072699 128.449152) (width 1) (layer "B.Cu") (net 18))
 (segment (start 130.175 122.022056) (end 130.175 128.905) (width 1) (layer "B.Cu") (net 18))
 (segment (start 130.36924 121.827816) (end 130.175 122.022056) (width 1) (layer "B.Cu") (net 18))
 (segment (start 108 73.96) (end 130.36924 96.32924) (width 1) (layer "B.Cu") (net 18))
 (segment (start 130.175 128.905) (end 138.616851 128.905) (width 1) (layer "B.Cu") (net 18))
 (segment (start 130.36924 96.32924) (end 130.36924 121.827816) (width 1) (layer "B.Cu") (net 18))
 (segment (start 136.604375 117.804375) (end 136.604375 120.336607) (width 1) (layer "F.Cu") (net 21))
 (segment (start 108 89.2) (end 136.604375 117.804375) (width 1) (layer "F.Cu") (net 21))
 (segment (start 138.0725 123.785) (end 135.785 123.785) (width 0.4) (layer "F.Cu") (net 21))
 (segment (start 135.785 123.785) (end 134.5 122.5) (width 0.4) (layer "F.Cu") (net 21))
 (via (at 134.5 122.5) (size 0.6) (drill 0.3) (layers "F.Cu" "B.Cu") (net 21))
 (via (at 136.604375 120.336607) (size 0.6) (drill 0.3) (layers "F.Cu" "B.Cu") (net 21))
 (segment (start 134.5 122.5) (end 136.604375 120.395625) (width 1) (layer "B.Cu") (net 21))
 (segment (start 136.604375 120.395625) (end 136.604375 120.336607) (width 1) (layer "B.Cu") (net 21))
 (segment (start 128 124) (end 128.4 124.4) (width 0.4) (layer "F.Cu") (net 24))
 (segment (start 125.02 124) (end 128 124) (width 1) (layer "F.Cu") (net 24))
 (segment (start 128.4 124.4) (end 130.935122 124.4) (width 0.4) (layer "F.Cu") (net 24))
 (segment (start 131.550122 123.785) (end 132.3475 123.785) (width 0.4) (layer "F.Cu") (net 24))
 (segment (start 108 106.98) (end 125.02 124) (width 1) (layer "F.Cu") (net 24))
 (segment (start 130.935122 124.4) (end 131.550122 123.785) (width 0.4) (layer "F.Cu") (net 24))
 (segment (start 131.351594 126.385) (end 132.3475 126.385) (width 0.4) (layer "F.Cu") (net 27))
 (segment (start 131.236594 126.5) (end 131.351594 126.385) (width 0.4) (layer "F.Cu") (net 27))
 (segment (start 117.56 126.7) (end 130.3 126.7) (width 1) (layer "F.Cu") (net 27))
 (segment (start 108 117.14) (end 117.56 126.7) (width 1) (layer "F.Cu") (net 27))
 (segment (start 130.5 126.5) (end 131.236594 126.5) (width 0.4) (layer "F.Cu") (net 27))
 (segment (start 130.3 126.7) (end 130.5 126.5) (width 1) (layer "F.Cu") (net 27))
 (segment (start 131.515 122.485) (end 130.5 123.5) (width 0.4) (layer "F.Cu") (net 23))
 (segment (start 129.6 123.5) (end 108 101.9) (width 1) (layer "F.Cu") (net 23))
 (segment (start 132.3475 122.485) (end 131.515 122.485) (width 0.4) (layer "F.Cu") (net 23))
 (segment (start 130.5 123.5) (end 129.6 123.5) (width 1) (layer "F.Cu") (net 23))
 (segment (start 179.815 138.95) (end 167.465 126.6) (width 1) (layer "F.Cu") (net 6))
 (segment (start 141.4 126.6) (end 141 127) (width 1) (layer "F.Cu") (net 6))
 (segment (start 141 127) (end 140.965 127.035) (width 0.4) (layer "F.Cu") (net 6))
 (segment (start 140.965 127.035) (end 138.0725 127.035) (width 0.4) (layer "F.Cu") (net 6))
 (segment (start 167.465 126.6) (end 141.4 126.6) (width 1) (layer "F.Cu") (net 6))
 (segment (start 201.53 140.287081) (end 201.53 132.66) (width 1) (layer "F.Cu") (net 2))
 (segment (start 132.892378 120.9325) (end 131.910613 120.9325) (width 0.4) (layer "F.Cu") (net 2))
 (segment (start 133.485 122.794878) (end 133.485 121.525122) (width 0.4) (layer "F.Cu") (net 2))
 (segment (start 200.625581 131.755581) (end 200.625581 130.072) (width 1) (layer "F.Cu") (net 2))
 (segment (start 133.485 121.525122) (end 132.892378 120.9325) (width 0.4) (layer "F.Cu") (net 2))
 (segment (start 133.144878 123.135) (end 133.485 122.794878) (width 0.4) (layer "F.Cu") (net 2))
 (segment (start 132.3475 123.135) (end 133.144878 123.135) (width 0.4) (layer "F.Cu") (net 2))
 (segment (start 199.98 126.03) (end 199.98 119.125) (width 1) (layer "F.Cu") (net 2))
 (segment (start 201.482 129.215581) (end 201.482 127.532) (width 1) (layer "F.Cu") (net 2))
 (segment (start 201.53 132.66) (end 200.625581 131.755581) (width 1) (layer "F.Cu") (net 2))
 (segment (start 201.482 127.532) (end 199.98 126.03) (width 1) (layer "F.Cu") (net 2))
 (segment (start 199.98 140.635) (end 201.182081 140.635) (width 1) (layer "F.Cu") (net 2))
 (segment (start 200.625581 130.072) (end 201.482 129.215581) (width 1) (layer "F.Cu") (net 2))
 (segment (start 201.182081 140.635) (end 201.53 140.287081) (width 1) (layer "F.Cu") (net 2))
 (segment (start 131.910613 120.9325) (end 131.601404 120.623291) (width 0.4) (layer "F.Cu") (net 2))
 (via (at 131.601404 120.623291) (size 0.6) (drill 0.3) (layers "F.Cu" "B.Cu") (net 2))
 (segment (start 133.099695 119.125) (end 131.601404 120.623291) (width 1) (layer "B.Cu") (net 2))
 (segment (start 199.98 119.125) (end 133.099695 119.125) (width 1) (layer "B.Cu") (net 2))
 (segment (start 134.62 127) (end 134.62 128.27) (width 1) (layer "F.Cu") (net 1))
 (segment (start 136.93 130.58) (end 137.741321 130.58) (width 1) (layer "F.Cu") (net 1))
 (segment (start 155.956574 131.7) (end 156.006574 131.75) (width 1) (layer "F.Cu") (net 1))
 (segment (start 138.861321 131.7) (end 155.956574 131.7) (width 1) (layer "F.Cu") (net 1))
 (segment (start 132.3475 125.735) (end 133.355 125.735) (width 0.4) (layer "F.Cu") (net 1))
 (segment (start 199.98 138.095) (end 199.258001 137.373001) (width 1) (layer "F.Cu") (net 1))
 (segment (start 199.258001 129.371999) (end 200.02 128.61) (width 1) (layer "F.Cu") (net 1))
 (segment (start 137.741321 130.58) (end 138.861321 131.7) (width 1) (layer "F.Cu") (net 1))
 (segment (start 133.355 125.735) (end 134.62 127) (width 0.4) (layer "F.Cu") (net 1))
 (segment (start 199.258001 137.373001) (end 199.258001 129.371999) (width 1) (layer "F.Cu") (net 1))
 (segment (start 134.62 128.27) (end 136.93 130.58) (width 1) (layer "F.Cu") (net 1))
 (via (at 156.006574 131.75) (size 0.5) (drill 0.3) (layers "F.Cu" "B.Cu") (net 1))
 (segment (start 159.146574 128.61) (end 156.006574 131.75) (width 1) (layer "B.Cu") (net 1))
 (segment (start 200.02 128.61) (end 159.146574 128.61) (width 1) (layer "B.Cu") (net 1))
 (segment (start 167.014145 128.439145) (end 140.426209 128.439145) (width 1) (layer "F.Cu") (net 7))
 (segment (start 177.525 138.95) (end 167.014145 128.439145) (width 1) (layer "F.Cu") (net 7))
 (segment (start 140.426209 128.439145) (end 139.466202 129.399152) (width 1) (layer "F.Cu") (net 7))
 (segment (start 138.679196 129.399152) (end 138.629196 129.349152) (width 1) (layer "F.Cu") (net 7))
 (segment (start 136.065 124.435) (end 135.5 125) (width 0.4) (layer "F.Cu") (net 7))
 (segment (start 137.849152 129.349152) (end 135.88747 127.38747) (width 1) (layer "F.Cu") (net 7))
 (segment (start 138.629196 129.349152) (end 137.849152 129.349152) (width 1) (layer "F.Cu") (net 7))
 (segment (start 135.88747 126.38747) (end 135.88747 127.38747) (width 1) (layer "F.Cu") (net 7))
 (segment (start 135.5 125) (end 135.5 126) (width 1) (layer "F.Cu") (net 7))
 (segment (start 135.5 126) (end 135.88747 126.38747) (width 1) (layer "F.Cu") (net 7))
 (segment (start 138.0725 124.435) (end 136.065 124.435) (width 0.4) (layer "F.Cu") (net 7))
 (segment (start 139.466202 129.399152) (end 138.679196 129.399152) (width 1) (layer "F.Cu") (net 7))
 (segment (start 136.93747 125.949634) (end 137.152104 125.735) (width 0.4) (layer "F.Cu") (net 8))
 (segment (start 165.924145 129.639145) (end 141.093087 129.639145) (width 1) (layer "F.Cu") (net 8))
 (segment (start 137.152104 125.735) (end 138.0725 125.735) (width 0.4) (layer "F.Cu") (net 8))
 (segment (start 175.235 138.95) (end 165.924145 129.639145) (width 1) (layer "F.Cu") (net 8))
 (via (at 136.93747 125.949634) (size 0.6) (drill 0.3) (layers "F.Cu" "B.Cu") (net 8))
 (via (at 141.093087 129.639145) (size 0.6) (drill 0.3) (layers "F.Cu" "B.Cu") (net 8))
 (segment (start 138.287134 125.949634) (end 141.093087 128.755587) (width 1) (layer "B.Cu") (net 8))
 (segment (start 141.093087 128.755587) (end 141.093087 129.639145) (width 1) (layer "B.Cu") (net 8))
 (segment (start 136.93747 125.949634) (end 138.287134 125.949634) (width 1) (layer "B.Cu") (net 8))
 (segment (start 127.08 137.875) (end 137.08 137.875) (width 1) (layer "F.Cu") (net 3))
 (segment (start 152.568001 122.386999) (end 201.718001 122.386999) (width 1) (layer "B.Cu") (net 3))
 (segment (start 137.08 137.875) (end 152.568001 122.386999) (width 1) (layer "B.Cu") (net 3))
 (segment (start 201.718001 122.386999) (end 202.48 121.625) (width 1) (layer "B.Cu") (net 3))
 (segment (start 130.5 122) (end 131.151472 122) (width 0.4) (layer "F.Cu") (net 14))
 (segment (start 129.83848 122) (end 129.16924 121.33076) (width 1) (layer "F.Cu") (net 14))
 (segment (start 130.5 122) (end 129.83848 122) (width 1) (layer "F.Cu") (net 14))
 (segment (start 131.266472 121.885) (end 131.548972 121.885) (width 0.4) (layer "F.Cu") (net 14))
 (segment (start 131.151472 122) (end 131.266472 121.885) (width 0.4) (layer "F.Cu") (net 14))
 (via (at 129.16924 121.33076) (size 0.6) (drill 0.3) (layers "F.Cu" "B.Cu") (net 14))
 (segment (start 172.945 142.91) (end 171.01 144.845) (width 1) (layer "B.Cu") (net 14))
 (segment (start 171.01 144.845) (end 140.345 144.845) (width 1) (layer "B.Cu") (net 14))
 (segment (start 140.345 144.845) (end 128.633884 133.133884) (width 1) (layer "B.Cu") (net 14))
 (segment (start 128.633884 121.866116) (end 129.16924 121.33076) (width 1) (layer "B.Cu") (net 14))
 (segment (start 128.633884 133.133884) (end 128.633884 121.866116) (width 1) (layer "B.Cu") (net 14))
 (segment (start 136.135 123.135) (end 138.0725 123.135) (width 0.4) (layer "F.Cu") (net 13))
 (segment (start 173.735 144.41) (end 167.991623 144.41) (width 1) (layer "F.Cu") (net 13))
 (segment (start 159.318377 133.5) (end 139 133.5) (width 1) (layer "F.Cu") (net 13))
 (segment (start 167.991623 144.41) (end 167.991623 142.173246) (width 1) (layer "F.Cu") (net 13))
 (segment (start 175.235 142.91) (end 173.735 144.41) (width 1) (layer "F.Cu") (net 13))
 (segment (start 167.991623 142.173246) (end 159.318377 133.5) (width 1) (layer "F.Cu") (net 13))
 (segment (start 136 123) (end 136.135 123.135) (width 0.4) (layer "F.Cu") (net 13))
 (via (at 139 133.5) (size 0.6) (drill 0.3) (layers "F.Cu" "B.Cu") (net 13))
 (via (at 136 123) (size 0.6) (drill 0.3) (layers "F.Cu" "B.Cu") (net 13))
 (segment (start 138 123.5) (end 137.5 123) (width 1) (layer "B.Cu") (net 13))
 (segment (start 143.5 129) (end 138 123.5) (width 1) (layer "B.Cu") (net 13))
 (segment (start 137.5 123) (end 136 123) (width 1) (layer "B.Cu") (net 13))
 (segment (start 139 133.5) (end 143.5 129) (width 1) (layer "B.Cu") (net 13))
 (segment (start 142.32 137.795) (end 152.32 137.795) (width 1) (layer "F.Cu") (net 5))
 (segment (start 152.32 137.795) (end 156.765 133.35) (width 1) (layer "B.Cu") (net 5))
 (segment (start 200.28 133.35) (end 202.52 131.11) (width 1) (layer "B.Cu") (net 5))
 (segment (start 156.765 133.35) (end 200.28 133.35) (width 1) (layer "B.Cu") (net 5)))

